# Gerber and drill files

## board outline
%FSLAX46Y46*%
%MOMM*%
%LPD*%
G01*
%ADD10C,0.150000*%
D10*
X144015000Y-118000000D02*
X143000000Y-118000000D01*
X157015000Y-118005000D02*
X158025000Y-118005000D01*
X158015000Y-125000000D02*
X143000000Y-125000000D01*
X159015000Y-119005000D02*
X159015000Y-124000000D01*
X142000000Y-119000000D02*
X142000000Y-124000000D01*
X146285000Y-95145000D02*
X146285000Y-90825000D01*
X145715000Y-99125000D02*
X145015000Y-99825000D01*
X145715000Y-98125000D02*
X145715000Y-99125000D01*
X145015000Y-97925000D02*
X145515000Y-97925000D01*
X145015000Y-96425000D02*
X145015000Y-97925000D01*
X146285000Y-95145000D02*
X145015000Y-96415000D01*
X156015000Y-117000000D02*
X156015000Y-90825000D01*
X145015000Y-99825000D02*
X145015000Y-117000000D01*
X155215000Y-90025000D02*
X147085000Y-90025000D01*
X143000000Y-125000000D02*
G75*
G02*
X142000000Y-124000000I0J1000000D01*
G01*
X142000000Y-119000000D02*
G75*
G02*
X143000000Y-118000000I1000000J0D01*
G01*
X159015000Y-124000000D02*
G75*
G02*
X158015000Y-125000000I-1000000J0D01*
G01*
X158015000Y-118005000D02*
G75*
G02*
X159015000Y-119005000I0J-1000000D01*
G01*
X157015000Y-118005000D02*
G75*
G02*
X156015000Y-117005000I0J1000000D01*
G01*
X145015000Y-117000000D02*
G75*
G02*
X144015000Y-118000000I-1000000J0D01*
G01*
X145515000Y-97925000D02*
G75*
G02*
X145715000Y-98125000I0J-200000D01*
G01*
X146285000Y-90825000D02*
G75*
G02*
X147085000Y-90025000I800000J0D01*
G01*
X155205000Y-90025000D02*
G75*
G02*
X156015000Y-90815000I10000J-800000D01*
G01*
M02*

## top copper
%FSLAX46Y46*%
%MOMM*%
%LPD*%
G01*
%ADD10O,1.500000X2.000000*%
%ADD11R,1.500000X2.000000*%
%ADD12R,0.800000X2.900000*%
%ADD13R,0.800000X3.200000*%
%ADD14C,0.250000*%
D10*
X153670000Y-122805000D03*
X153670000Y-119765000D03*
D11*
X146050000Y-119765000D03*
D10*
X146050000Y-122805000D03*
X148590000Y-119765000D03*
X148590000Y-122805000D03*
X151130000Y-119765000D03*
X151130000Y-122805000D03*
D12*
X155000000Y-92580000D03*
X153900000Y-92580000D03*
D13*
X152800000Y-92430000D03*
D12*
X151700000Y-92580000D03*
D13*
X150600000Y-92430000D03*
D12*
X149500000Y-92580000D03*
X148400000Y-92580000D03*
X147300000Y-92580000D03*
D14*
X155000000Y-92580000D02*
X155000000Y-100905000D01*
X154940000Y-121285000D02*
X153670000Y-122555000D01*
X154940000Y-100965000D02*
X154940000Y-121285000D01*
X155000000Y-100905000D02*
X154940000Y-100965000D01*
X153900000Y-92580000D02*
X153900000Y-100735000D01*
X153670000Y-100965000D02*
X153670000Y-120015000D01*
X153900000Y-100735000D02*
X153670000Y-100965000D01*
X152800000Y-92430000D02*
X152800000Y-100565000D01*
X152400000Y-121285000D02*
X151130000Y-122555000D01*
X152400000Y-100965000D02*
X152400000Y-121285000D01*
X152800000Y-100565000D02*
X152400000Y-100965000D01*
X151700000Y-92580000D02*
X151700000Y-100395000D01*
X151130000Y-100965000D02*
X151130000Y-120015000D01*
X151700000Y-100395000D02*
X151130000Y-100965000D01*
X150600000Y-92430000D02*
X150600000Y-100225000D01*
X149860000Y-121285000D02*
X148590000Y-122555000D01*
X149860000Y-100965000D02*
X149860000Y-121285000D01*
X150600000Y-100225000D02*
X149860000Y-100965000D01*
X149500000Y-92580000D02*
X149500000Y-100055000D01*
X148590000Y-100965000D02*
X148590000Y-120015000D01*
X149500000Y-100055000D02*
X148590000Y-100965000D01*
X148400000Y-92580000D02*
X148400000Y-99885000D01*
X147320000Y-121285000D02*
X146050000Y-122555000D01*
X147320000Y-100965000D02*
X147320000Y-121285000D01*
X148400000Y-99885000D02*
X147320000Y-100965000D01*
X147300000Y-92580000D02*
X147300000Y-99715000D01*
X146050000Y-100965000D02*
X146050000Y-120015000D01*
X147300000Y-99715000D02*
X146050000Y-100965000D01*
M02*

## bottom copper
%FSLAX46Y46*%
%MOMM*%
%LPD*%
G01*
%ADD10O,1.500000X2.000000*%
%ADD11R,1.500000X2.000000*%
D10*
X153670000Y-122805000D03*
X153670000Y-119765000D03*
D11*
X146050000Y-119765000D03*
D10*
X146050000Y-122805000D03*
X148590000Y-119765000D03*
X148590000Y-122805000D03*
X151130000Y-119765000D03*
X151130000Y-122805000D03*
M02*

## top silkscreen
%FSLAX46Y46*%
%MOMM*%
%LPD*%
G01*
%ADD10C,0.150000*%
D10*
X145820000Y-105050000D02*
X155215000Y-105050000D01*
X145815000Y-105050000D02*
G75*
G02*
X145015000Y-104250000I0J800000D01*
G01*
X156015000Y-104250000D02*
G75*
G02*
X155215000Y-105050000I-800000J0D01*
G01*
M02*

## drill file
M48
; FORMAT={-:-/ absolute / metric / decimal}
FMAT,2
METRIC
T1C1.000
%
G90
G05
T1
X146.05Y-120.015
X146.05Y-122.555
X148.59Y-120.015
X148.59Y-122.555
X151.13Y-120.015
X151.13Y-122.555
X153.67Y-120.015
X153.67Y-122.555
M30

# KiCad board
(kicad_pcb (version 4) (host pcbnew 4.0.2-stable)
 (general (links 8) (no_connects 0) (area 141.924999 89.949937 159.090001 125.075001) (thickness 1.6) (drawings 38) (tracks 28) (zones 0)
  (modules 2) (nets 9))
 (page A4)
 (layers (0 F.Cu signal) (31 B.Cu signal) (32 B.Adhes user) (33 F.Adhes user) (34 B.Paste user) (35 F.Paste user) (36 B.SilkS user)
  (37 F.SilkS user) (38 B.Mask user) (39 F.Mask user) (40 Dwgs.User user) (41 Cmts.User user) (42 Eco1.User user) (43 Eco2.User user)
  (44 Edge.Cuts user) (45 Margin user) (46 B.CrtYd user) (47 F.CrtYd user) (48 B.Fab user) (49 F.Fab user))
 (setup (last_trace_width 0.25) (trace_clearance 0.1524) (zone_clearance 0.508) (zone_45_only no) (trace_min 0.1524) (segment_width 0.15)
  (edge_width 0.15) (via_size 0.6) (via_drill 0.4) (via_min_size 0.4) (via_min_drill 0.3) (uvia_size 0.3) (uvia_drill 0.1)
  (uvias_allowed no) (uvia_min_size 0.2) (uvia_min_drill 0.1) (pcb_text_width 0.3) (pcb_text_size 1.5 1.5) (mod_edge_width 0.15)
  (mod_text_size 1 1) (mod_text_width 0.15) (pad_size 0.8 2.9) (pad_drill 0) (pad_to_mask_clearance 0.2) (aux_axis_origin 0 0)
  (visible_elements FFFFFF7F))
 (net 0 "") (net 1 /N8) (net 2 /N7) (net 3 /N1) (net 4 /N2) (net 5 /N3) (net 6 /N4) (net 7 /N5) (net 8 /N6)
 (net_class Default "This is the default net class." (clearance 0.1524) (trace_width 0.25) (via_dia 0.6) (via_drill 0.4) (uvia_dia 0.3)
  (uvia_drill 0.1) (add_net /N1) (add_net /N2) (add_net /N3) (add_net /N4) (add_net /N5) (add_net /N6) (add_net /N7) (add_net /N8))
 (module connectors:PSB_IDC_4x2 (layer B.Cu) (at 149.86 121.285)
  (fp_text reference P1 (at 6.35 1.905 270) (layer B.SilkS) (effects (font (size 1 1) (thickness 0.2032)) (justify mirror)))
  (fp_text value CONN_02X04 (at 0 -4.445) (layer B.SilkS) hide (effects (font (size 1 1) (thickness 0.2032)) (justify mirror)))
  (pad 8 thru_hole oval (at 3.81 1.27) (size 1.5 2) (drill 1 (offset 0 0.25)) (layers *.Cu *.Mask B.SilkS) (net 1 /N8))
  (pad 7 thru_hole oval (at 3.81 -1.27) (size 1.5 2) (drill 1 (offset 0 -0.25)) (layers *.Cu *.Mask B.SilkS) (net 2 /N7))
  (pad 1 thru_hole rect (at -3.81 -1.27) (size 1.5 2) (drill 1 (offset 0 -0.25)) (layers *.Cu *.Mask B.SilkS) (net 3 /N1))
  (pad 2 thru_hole oval (at -3.81 1.27) (size 1.5 2) (drill 1 (offset 0 0.25)) (layers *.Cu *.Mask B.SilkS) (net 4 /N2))
  (pad 3 thru_hole oval (at -1.27 -1.27) (size 1.5 2) (drill 1 (offset 0 -0.25)) (layers *.Cu *.Mask B.SilkS) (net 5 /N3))
  (pad 4 thru_hole oval (at -1.27 1.27) (size 1.5 2) (drill 1 (offset 0 0.25)) (layers *.Cu *.Mask B.SilkS) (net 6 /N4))
  (pad 5 thru_hole oval (at 1.27 -1.27) (size 1.5 2) (drill 1 (offset 0 -0.25)) (layers *.Cu *.Mask B.SilkS) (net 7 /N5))
  (pad 6 thru_hole oval (at 1.27 1.27) (size 1.5 2) (drill 1 (offset 0 0.25)) (layers *.Cu *.Mask B.SilkS) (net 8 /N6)))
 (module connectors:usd (layer F.Cu) (at 147.3 92.58)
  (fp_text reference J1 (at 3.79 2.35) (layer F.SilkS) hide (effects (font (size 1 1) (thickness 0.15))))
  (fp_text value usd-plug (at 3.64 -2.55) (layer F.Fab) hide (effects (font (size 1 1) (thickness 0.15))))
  (pad 8 smd rect (at 7.7 0) (size 0.8 2.9) (layers F.Cu F.Paste F.Mask) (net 1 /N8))
  (pad 7 smd rect (at 6.6 0) (size 0.8 2.9) (layers F.Cu F.Paste F.Mask) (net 2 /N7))
  (pad 6 smd rect (at 5.5 -0.15) (size 0.8 3.2) (layers F.Cu F.Paste F.Mask) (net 8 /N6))
  (pad 5 smd rect (at 4.4 0) (size 0.8 2.9) (layers F.Cu F.Paste F.Mask) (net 7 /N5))
  (pad 4 smd rect (at 3.3 -0.15) (size 0.8 3.2) (layers F.Cu F.Paste F.Mask) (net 6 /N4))
  (pad 3 smd rect (at 2.2 0) (size 0.8 2.9) (layers F.Cu F.Paste F.Mask) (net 5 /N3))
  (pad 2 smd rect (at 1.1 0) (size 0.8 2.9) (layers F.Cu F.Paste F.Mask) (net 4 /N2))
  (pad 1 smd rect (at 0 0) (size 0.8 2.9) (layers F.Cu F.Paste F.Mask) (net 3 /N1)))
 (gr_line (start 144.015 118) (end 143 118) (angle 90) (layer Edge.Cuts) (width 0.15))
 (gr_line (start 157.015 118.005) (end 158.025 118.005) (angle 90) (layer Edge.Cuts) (width 0.15))
 (gr_line (start 158.015 125) (end 143 125) (angle 90) (layer Edge.Cuts) (width 0.15))
 (gr_line (start 159.015 119.005) (end 159.015 124) (angle 90) (layer Edge.Cuts) (width 0.15))
 (gr_line (start 142 119) (end 142 124) (angle 90) (layer Edge.Cuts) (width 0.15))
 (gr_line (start 145.82 105.05) (end 155.215 105.05) (angle 90) (layer F.SilkS) (width 0.15))
 (gr_line (start 146.285 95.145) (end 146.285 90.825) (angle 90) (layer Edge.Cuts) (width 0.15))
 (gr_line (start 145.715 99.125) (end 145.015 99.825) (angle 90) (layer Edge.Cuts) (width 0.15))
 (gr_line (start 145.715 98.125) (end 145.715 99.125) (angle 90) (layer Edge.Cuts) (width 0.15))
 (gr_line (start 145.015 97.925) (end 145.515 97.925) (angle 90) (layer Edge.Cuts) (width 0.15))
 (gr_line (start 145.015 96.425) (end 145.015 97.925) (angle 90) (layer Edge.Cuts) (width 0.15))
 (gr_line (start 146.285 95.145) (end 145.015 96.415) (angle 90) (layer Edge.Cuts) (width 0.15))
 (gr_line (start 156.015 117) (end 156.015 90.825) (angle 90) (layer Edge.Cuts) (width 0.15))
 (gr_line (start 145.015 99.825) (end 145.015 117) (angle 90) (layer Edge.Cuts) (width 0.15))
 (gr_line (start 155.215 90.025) (end 147.085 90.025) (angle 90) (layer Edge.Cuts) (width 0.15))
 (gr_arc (start 143 124) (end 143 125) (angle 90) (layer Edge.Cuts) (width 0.15))
 (gr_arc (start 143 119) (end 142 119) (angle 90) (layer Edge.Cuts) (width 0.15))
 (gr_arc (start 158.015 124) (end 159.015 124) (angle 90) (layer Edge.Cuts) (width 0.15))
 (gr_arc (start 158.015 119.005) (end 158.015 118.005) (angle 90) (layer Edge.Cuts) (width 0.15))
 (gr_arc (start 157.015 117.005) (end 157.015 118.005) (angle 90) (layer Edge.Cuts) (width 0.15))
 (gr_arc (start 144.015 117) (end 145.015 117) (angle 90) (layer Edge.Cuts) (width 0.15))
 (gr_arc (start 145.815 104.25) (end 145.815 105.05) (angle 90) (layer F.SilkS) (width 0.15))
 (gr_arc (start 155.215 104.25) (end 156.015 104.25) (angle 90) (layer F.SilkS) (width 0.15))
 (gr_arc (start 145.515 98.125) (end 145.715 98.125) (angle -90) (layer Edge.Cuts) (width 0.15))
 (gr_arc (start 147.085 90.825) (end 147.085 90.025) (angle -90) (layer Edge.Cuts) (width 0.15))
 (gr_arc (start 155.215 90.825) (end 156.015 90.815) (angle -90) (layer Edge.Cuts) (width 0.15))
 (segment (start 155 92.58) (end 155 100.905) (width 0.25) (layer F.Cu) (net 1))
 (segment (start 154.94 121.285) (end 153.67 122.555) (width 0.25) (layer F.Cu) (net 1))
 (segment (start 154.94 100.965) (end 154.94 121.285) (width 0.25) (layer F.Cu) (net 1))
 (segment (start 155 100.905) (end 154.94 100.965) (width 0.25) (layer F.Cu) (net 1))
 (segment (start 153.9 92.58) (end 153.9 100.735) (width 0.25) (layer F.Cu) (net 2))
 (segment (start 153.67 100.965) (end 153.67 120.015) (width 0.25) (layer F.Cu) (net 2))
 (segment (start 153.9 100.735) (end 153.67 100.965) (width 0.25) (layer F.Cu) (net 2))
 (segment (start 152.8 92.43) (end 152.8 100.565) (width 0.25) (layer F.Cu) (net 8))
 (segment (start 152.4 121.285) (end 151.13 122.555) (width 0.25) (layer F.Cu) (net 8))
 (segment (start 152.4 100.965) (end 152.4 121.285) (width 0.25) (layer F.Cu) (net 8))
 (segment (start 152.8 100.565) (end 152.4 100.965) (width 0.25) (layer F.Cu) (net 8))
 (segment (start 151.7 92.58) (end 151.7 100.395) (width 0.25) (layer F.Cu) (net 7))
 (segment (start 151.13 100.965) (end 151.13 120.015) (width 0.25) (layer F.Cu) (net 7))
 (segment (start 151.7 100.395) (end 151.13 100.965) (width 0.25) (layer F.Cu) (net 7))
 (segment (start 150.6 92.43) (end 150.6 100.225) (width 0.25) (layer F.Cu) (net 6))
 (segment (start 149.86 121.285) (end 148.59 122.555) (width 0.25) (layer F.Cu) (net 6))
 (segment (start 149.86 100.965) (end 149.86 121.285) (width 0.25) (layer F.Cu) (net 6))
 (segment (start 150.6 100.225) (end 149.86 100.965) (width 0.25) (layer F.Cu) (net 6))
 (segment (start 149.5 92.58) (end 149.5 100.055) (width 0.25) (layer F.Cu) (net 5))
 (segment (start 148.59 100.965) (end 148.59 120.015) (width 0.25) (layer F.Cu) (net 5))
 (segment (start 149.5 100.055) (end 148.59 100.965) (width 0.25) (layer F.Cu) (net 5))
 (segment (start 148.4 92.58) (end 148.4 99.885) (width 0.25) (layer F.Cu) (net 4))
 (segment (start 147.32 121.285) (end 146.05 122.555) (width 0.25) (layer F.Cu) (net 4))
 (segment (start 147.32 100.965) (end 147.32 121.285) (width 0.25) (layer F.Cu) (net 4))
 (segment (start 148.4 99.885) (end 147.32 100.965) (width 0.25) (layer F.Cu) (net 4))
 (segment (start 147.3 92.58) (end 147.3 99.715) (width 0.25) (layer F.Cu) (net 3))
 (segment (start 146.05 100.965) (end 146.05 120.015) (width 0.25) (layer F.Cu) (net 3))
 (segment (start 147.3 99.715) (end 146.05 100.965) (width 0.25) (layer F.Cu) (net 3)))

